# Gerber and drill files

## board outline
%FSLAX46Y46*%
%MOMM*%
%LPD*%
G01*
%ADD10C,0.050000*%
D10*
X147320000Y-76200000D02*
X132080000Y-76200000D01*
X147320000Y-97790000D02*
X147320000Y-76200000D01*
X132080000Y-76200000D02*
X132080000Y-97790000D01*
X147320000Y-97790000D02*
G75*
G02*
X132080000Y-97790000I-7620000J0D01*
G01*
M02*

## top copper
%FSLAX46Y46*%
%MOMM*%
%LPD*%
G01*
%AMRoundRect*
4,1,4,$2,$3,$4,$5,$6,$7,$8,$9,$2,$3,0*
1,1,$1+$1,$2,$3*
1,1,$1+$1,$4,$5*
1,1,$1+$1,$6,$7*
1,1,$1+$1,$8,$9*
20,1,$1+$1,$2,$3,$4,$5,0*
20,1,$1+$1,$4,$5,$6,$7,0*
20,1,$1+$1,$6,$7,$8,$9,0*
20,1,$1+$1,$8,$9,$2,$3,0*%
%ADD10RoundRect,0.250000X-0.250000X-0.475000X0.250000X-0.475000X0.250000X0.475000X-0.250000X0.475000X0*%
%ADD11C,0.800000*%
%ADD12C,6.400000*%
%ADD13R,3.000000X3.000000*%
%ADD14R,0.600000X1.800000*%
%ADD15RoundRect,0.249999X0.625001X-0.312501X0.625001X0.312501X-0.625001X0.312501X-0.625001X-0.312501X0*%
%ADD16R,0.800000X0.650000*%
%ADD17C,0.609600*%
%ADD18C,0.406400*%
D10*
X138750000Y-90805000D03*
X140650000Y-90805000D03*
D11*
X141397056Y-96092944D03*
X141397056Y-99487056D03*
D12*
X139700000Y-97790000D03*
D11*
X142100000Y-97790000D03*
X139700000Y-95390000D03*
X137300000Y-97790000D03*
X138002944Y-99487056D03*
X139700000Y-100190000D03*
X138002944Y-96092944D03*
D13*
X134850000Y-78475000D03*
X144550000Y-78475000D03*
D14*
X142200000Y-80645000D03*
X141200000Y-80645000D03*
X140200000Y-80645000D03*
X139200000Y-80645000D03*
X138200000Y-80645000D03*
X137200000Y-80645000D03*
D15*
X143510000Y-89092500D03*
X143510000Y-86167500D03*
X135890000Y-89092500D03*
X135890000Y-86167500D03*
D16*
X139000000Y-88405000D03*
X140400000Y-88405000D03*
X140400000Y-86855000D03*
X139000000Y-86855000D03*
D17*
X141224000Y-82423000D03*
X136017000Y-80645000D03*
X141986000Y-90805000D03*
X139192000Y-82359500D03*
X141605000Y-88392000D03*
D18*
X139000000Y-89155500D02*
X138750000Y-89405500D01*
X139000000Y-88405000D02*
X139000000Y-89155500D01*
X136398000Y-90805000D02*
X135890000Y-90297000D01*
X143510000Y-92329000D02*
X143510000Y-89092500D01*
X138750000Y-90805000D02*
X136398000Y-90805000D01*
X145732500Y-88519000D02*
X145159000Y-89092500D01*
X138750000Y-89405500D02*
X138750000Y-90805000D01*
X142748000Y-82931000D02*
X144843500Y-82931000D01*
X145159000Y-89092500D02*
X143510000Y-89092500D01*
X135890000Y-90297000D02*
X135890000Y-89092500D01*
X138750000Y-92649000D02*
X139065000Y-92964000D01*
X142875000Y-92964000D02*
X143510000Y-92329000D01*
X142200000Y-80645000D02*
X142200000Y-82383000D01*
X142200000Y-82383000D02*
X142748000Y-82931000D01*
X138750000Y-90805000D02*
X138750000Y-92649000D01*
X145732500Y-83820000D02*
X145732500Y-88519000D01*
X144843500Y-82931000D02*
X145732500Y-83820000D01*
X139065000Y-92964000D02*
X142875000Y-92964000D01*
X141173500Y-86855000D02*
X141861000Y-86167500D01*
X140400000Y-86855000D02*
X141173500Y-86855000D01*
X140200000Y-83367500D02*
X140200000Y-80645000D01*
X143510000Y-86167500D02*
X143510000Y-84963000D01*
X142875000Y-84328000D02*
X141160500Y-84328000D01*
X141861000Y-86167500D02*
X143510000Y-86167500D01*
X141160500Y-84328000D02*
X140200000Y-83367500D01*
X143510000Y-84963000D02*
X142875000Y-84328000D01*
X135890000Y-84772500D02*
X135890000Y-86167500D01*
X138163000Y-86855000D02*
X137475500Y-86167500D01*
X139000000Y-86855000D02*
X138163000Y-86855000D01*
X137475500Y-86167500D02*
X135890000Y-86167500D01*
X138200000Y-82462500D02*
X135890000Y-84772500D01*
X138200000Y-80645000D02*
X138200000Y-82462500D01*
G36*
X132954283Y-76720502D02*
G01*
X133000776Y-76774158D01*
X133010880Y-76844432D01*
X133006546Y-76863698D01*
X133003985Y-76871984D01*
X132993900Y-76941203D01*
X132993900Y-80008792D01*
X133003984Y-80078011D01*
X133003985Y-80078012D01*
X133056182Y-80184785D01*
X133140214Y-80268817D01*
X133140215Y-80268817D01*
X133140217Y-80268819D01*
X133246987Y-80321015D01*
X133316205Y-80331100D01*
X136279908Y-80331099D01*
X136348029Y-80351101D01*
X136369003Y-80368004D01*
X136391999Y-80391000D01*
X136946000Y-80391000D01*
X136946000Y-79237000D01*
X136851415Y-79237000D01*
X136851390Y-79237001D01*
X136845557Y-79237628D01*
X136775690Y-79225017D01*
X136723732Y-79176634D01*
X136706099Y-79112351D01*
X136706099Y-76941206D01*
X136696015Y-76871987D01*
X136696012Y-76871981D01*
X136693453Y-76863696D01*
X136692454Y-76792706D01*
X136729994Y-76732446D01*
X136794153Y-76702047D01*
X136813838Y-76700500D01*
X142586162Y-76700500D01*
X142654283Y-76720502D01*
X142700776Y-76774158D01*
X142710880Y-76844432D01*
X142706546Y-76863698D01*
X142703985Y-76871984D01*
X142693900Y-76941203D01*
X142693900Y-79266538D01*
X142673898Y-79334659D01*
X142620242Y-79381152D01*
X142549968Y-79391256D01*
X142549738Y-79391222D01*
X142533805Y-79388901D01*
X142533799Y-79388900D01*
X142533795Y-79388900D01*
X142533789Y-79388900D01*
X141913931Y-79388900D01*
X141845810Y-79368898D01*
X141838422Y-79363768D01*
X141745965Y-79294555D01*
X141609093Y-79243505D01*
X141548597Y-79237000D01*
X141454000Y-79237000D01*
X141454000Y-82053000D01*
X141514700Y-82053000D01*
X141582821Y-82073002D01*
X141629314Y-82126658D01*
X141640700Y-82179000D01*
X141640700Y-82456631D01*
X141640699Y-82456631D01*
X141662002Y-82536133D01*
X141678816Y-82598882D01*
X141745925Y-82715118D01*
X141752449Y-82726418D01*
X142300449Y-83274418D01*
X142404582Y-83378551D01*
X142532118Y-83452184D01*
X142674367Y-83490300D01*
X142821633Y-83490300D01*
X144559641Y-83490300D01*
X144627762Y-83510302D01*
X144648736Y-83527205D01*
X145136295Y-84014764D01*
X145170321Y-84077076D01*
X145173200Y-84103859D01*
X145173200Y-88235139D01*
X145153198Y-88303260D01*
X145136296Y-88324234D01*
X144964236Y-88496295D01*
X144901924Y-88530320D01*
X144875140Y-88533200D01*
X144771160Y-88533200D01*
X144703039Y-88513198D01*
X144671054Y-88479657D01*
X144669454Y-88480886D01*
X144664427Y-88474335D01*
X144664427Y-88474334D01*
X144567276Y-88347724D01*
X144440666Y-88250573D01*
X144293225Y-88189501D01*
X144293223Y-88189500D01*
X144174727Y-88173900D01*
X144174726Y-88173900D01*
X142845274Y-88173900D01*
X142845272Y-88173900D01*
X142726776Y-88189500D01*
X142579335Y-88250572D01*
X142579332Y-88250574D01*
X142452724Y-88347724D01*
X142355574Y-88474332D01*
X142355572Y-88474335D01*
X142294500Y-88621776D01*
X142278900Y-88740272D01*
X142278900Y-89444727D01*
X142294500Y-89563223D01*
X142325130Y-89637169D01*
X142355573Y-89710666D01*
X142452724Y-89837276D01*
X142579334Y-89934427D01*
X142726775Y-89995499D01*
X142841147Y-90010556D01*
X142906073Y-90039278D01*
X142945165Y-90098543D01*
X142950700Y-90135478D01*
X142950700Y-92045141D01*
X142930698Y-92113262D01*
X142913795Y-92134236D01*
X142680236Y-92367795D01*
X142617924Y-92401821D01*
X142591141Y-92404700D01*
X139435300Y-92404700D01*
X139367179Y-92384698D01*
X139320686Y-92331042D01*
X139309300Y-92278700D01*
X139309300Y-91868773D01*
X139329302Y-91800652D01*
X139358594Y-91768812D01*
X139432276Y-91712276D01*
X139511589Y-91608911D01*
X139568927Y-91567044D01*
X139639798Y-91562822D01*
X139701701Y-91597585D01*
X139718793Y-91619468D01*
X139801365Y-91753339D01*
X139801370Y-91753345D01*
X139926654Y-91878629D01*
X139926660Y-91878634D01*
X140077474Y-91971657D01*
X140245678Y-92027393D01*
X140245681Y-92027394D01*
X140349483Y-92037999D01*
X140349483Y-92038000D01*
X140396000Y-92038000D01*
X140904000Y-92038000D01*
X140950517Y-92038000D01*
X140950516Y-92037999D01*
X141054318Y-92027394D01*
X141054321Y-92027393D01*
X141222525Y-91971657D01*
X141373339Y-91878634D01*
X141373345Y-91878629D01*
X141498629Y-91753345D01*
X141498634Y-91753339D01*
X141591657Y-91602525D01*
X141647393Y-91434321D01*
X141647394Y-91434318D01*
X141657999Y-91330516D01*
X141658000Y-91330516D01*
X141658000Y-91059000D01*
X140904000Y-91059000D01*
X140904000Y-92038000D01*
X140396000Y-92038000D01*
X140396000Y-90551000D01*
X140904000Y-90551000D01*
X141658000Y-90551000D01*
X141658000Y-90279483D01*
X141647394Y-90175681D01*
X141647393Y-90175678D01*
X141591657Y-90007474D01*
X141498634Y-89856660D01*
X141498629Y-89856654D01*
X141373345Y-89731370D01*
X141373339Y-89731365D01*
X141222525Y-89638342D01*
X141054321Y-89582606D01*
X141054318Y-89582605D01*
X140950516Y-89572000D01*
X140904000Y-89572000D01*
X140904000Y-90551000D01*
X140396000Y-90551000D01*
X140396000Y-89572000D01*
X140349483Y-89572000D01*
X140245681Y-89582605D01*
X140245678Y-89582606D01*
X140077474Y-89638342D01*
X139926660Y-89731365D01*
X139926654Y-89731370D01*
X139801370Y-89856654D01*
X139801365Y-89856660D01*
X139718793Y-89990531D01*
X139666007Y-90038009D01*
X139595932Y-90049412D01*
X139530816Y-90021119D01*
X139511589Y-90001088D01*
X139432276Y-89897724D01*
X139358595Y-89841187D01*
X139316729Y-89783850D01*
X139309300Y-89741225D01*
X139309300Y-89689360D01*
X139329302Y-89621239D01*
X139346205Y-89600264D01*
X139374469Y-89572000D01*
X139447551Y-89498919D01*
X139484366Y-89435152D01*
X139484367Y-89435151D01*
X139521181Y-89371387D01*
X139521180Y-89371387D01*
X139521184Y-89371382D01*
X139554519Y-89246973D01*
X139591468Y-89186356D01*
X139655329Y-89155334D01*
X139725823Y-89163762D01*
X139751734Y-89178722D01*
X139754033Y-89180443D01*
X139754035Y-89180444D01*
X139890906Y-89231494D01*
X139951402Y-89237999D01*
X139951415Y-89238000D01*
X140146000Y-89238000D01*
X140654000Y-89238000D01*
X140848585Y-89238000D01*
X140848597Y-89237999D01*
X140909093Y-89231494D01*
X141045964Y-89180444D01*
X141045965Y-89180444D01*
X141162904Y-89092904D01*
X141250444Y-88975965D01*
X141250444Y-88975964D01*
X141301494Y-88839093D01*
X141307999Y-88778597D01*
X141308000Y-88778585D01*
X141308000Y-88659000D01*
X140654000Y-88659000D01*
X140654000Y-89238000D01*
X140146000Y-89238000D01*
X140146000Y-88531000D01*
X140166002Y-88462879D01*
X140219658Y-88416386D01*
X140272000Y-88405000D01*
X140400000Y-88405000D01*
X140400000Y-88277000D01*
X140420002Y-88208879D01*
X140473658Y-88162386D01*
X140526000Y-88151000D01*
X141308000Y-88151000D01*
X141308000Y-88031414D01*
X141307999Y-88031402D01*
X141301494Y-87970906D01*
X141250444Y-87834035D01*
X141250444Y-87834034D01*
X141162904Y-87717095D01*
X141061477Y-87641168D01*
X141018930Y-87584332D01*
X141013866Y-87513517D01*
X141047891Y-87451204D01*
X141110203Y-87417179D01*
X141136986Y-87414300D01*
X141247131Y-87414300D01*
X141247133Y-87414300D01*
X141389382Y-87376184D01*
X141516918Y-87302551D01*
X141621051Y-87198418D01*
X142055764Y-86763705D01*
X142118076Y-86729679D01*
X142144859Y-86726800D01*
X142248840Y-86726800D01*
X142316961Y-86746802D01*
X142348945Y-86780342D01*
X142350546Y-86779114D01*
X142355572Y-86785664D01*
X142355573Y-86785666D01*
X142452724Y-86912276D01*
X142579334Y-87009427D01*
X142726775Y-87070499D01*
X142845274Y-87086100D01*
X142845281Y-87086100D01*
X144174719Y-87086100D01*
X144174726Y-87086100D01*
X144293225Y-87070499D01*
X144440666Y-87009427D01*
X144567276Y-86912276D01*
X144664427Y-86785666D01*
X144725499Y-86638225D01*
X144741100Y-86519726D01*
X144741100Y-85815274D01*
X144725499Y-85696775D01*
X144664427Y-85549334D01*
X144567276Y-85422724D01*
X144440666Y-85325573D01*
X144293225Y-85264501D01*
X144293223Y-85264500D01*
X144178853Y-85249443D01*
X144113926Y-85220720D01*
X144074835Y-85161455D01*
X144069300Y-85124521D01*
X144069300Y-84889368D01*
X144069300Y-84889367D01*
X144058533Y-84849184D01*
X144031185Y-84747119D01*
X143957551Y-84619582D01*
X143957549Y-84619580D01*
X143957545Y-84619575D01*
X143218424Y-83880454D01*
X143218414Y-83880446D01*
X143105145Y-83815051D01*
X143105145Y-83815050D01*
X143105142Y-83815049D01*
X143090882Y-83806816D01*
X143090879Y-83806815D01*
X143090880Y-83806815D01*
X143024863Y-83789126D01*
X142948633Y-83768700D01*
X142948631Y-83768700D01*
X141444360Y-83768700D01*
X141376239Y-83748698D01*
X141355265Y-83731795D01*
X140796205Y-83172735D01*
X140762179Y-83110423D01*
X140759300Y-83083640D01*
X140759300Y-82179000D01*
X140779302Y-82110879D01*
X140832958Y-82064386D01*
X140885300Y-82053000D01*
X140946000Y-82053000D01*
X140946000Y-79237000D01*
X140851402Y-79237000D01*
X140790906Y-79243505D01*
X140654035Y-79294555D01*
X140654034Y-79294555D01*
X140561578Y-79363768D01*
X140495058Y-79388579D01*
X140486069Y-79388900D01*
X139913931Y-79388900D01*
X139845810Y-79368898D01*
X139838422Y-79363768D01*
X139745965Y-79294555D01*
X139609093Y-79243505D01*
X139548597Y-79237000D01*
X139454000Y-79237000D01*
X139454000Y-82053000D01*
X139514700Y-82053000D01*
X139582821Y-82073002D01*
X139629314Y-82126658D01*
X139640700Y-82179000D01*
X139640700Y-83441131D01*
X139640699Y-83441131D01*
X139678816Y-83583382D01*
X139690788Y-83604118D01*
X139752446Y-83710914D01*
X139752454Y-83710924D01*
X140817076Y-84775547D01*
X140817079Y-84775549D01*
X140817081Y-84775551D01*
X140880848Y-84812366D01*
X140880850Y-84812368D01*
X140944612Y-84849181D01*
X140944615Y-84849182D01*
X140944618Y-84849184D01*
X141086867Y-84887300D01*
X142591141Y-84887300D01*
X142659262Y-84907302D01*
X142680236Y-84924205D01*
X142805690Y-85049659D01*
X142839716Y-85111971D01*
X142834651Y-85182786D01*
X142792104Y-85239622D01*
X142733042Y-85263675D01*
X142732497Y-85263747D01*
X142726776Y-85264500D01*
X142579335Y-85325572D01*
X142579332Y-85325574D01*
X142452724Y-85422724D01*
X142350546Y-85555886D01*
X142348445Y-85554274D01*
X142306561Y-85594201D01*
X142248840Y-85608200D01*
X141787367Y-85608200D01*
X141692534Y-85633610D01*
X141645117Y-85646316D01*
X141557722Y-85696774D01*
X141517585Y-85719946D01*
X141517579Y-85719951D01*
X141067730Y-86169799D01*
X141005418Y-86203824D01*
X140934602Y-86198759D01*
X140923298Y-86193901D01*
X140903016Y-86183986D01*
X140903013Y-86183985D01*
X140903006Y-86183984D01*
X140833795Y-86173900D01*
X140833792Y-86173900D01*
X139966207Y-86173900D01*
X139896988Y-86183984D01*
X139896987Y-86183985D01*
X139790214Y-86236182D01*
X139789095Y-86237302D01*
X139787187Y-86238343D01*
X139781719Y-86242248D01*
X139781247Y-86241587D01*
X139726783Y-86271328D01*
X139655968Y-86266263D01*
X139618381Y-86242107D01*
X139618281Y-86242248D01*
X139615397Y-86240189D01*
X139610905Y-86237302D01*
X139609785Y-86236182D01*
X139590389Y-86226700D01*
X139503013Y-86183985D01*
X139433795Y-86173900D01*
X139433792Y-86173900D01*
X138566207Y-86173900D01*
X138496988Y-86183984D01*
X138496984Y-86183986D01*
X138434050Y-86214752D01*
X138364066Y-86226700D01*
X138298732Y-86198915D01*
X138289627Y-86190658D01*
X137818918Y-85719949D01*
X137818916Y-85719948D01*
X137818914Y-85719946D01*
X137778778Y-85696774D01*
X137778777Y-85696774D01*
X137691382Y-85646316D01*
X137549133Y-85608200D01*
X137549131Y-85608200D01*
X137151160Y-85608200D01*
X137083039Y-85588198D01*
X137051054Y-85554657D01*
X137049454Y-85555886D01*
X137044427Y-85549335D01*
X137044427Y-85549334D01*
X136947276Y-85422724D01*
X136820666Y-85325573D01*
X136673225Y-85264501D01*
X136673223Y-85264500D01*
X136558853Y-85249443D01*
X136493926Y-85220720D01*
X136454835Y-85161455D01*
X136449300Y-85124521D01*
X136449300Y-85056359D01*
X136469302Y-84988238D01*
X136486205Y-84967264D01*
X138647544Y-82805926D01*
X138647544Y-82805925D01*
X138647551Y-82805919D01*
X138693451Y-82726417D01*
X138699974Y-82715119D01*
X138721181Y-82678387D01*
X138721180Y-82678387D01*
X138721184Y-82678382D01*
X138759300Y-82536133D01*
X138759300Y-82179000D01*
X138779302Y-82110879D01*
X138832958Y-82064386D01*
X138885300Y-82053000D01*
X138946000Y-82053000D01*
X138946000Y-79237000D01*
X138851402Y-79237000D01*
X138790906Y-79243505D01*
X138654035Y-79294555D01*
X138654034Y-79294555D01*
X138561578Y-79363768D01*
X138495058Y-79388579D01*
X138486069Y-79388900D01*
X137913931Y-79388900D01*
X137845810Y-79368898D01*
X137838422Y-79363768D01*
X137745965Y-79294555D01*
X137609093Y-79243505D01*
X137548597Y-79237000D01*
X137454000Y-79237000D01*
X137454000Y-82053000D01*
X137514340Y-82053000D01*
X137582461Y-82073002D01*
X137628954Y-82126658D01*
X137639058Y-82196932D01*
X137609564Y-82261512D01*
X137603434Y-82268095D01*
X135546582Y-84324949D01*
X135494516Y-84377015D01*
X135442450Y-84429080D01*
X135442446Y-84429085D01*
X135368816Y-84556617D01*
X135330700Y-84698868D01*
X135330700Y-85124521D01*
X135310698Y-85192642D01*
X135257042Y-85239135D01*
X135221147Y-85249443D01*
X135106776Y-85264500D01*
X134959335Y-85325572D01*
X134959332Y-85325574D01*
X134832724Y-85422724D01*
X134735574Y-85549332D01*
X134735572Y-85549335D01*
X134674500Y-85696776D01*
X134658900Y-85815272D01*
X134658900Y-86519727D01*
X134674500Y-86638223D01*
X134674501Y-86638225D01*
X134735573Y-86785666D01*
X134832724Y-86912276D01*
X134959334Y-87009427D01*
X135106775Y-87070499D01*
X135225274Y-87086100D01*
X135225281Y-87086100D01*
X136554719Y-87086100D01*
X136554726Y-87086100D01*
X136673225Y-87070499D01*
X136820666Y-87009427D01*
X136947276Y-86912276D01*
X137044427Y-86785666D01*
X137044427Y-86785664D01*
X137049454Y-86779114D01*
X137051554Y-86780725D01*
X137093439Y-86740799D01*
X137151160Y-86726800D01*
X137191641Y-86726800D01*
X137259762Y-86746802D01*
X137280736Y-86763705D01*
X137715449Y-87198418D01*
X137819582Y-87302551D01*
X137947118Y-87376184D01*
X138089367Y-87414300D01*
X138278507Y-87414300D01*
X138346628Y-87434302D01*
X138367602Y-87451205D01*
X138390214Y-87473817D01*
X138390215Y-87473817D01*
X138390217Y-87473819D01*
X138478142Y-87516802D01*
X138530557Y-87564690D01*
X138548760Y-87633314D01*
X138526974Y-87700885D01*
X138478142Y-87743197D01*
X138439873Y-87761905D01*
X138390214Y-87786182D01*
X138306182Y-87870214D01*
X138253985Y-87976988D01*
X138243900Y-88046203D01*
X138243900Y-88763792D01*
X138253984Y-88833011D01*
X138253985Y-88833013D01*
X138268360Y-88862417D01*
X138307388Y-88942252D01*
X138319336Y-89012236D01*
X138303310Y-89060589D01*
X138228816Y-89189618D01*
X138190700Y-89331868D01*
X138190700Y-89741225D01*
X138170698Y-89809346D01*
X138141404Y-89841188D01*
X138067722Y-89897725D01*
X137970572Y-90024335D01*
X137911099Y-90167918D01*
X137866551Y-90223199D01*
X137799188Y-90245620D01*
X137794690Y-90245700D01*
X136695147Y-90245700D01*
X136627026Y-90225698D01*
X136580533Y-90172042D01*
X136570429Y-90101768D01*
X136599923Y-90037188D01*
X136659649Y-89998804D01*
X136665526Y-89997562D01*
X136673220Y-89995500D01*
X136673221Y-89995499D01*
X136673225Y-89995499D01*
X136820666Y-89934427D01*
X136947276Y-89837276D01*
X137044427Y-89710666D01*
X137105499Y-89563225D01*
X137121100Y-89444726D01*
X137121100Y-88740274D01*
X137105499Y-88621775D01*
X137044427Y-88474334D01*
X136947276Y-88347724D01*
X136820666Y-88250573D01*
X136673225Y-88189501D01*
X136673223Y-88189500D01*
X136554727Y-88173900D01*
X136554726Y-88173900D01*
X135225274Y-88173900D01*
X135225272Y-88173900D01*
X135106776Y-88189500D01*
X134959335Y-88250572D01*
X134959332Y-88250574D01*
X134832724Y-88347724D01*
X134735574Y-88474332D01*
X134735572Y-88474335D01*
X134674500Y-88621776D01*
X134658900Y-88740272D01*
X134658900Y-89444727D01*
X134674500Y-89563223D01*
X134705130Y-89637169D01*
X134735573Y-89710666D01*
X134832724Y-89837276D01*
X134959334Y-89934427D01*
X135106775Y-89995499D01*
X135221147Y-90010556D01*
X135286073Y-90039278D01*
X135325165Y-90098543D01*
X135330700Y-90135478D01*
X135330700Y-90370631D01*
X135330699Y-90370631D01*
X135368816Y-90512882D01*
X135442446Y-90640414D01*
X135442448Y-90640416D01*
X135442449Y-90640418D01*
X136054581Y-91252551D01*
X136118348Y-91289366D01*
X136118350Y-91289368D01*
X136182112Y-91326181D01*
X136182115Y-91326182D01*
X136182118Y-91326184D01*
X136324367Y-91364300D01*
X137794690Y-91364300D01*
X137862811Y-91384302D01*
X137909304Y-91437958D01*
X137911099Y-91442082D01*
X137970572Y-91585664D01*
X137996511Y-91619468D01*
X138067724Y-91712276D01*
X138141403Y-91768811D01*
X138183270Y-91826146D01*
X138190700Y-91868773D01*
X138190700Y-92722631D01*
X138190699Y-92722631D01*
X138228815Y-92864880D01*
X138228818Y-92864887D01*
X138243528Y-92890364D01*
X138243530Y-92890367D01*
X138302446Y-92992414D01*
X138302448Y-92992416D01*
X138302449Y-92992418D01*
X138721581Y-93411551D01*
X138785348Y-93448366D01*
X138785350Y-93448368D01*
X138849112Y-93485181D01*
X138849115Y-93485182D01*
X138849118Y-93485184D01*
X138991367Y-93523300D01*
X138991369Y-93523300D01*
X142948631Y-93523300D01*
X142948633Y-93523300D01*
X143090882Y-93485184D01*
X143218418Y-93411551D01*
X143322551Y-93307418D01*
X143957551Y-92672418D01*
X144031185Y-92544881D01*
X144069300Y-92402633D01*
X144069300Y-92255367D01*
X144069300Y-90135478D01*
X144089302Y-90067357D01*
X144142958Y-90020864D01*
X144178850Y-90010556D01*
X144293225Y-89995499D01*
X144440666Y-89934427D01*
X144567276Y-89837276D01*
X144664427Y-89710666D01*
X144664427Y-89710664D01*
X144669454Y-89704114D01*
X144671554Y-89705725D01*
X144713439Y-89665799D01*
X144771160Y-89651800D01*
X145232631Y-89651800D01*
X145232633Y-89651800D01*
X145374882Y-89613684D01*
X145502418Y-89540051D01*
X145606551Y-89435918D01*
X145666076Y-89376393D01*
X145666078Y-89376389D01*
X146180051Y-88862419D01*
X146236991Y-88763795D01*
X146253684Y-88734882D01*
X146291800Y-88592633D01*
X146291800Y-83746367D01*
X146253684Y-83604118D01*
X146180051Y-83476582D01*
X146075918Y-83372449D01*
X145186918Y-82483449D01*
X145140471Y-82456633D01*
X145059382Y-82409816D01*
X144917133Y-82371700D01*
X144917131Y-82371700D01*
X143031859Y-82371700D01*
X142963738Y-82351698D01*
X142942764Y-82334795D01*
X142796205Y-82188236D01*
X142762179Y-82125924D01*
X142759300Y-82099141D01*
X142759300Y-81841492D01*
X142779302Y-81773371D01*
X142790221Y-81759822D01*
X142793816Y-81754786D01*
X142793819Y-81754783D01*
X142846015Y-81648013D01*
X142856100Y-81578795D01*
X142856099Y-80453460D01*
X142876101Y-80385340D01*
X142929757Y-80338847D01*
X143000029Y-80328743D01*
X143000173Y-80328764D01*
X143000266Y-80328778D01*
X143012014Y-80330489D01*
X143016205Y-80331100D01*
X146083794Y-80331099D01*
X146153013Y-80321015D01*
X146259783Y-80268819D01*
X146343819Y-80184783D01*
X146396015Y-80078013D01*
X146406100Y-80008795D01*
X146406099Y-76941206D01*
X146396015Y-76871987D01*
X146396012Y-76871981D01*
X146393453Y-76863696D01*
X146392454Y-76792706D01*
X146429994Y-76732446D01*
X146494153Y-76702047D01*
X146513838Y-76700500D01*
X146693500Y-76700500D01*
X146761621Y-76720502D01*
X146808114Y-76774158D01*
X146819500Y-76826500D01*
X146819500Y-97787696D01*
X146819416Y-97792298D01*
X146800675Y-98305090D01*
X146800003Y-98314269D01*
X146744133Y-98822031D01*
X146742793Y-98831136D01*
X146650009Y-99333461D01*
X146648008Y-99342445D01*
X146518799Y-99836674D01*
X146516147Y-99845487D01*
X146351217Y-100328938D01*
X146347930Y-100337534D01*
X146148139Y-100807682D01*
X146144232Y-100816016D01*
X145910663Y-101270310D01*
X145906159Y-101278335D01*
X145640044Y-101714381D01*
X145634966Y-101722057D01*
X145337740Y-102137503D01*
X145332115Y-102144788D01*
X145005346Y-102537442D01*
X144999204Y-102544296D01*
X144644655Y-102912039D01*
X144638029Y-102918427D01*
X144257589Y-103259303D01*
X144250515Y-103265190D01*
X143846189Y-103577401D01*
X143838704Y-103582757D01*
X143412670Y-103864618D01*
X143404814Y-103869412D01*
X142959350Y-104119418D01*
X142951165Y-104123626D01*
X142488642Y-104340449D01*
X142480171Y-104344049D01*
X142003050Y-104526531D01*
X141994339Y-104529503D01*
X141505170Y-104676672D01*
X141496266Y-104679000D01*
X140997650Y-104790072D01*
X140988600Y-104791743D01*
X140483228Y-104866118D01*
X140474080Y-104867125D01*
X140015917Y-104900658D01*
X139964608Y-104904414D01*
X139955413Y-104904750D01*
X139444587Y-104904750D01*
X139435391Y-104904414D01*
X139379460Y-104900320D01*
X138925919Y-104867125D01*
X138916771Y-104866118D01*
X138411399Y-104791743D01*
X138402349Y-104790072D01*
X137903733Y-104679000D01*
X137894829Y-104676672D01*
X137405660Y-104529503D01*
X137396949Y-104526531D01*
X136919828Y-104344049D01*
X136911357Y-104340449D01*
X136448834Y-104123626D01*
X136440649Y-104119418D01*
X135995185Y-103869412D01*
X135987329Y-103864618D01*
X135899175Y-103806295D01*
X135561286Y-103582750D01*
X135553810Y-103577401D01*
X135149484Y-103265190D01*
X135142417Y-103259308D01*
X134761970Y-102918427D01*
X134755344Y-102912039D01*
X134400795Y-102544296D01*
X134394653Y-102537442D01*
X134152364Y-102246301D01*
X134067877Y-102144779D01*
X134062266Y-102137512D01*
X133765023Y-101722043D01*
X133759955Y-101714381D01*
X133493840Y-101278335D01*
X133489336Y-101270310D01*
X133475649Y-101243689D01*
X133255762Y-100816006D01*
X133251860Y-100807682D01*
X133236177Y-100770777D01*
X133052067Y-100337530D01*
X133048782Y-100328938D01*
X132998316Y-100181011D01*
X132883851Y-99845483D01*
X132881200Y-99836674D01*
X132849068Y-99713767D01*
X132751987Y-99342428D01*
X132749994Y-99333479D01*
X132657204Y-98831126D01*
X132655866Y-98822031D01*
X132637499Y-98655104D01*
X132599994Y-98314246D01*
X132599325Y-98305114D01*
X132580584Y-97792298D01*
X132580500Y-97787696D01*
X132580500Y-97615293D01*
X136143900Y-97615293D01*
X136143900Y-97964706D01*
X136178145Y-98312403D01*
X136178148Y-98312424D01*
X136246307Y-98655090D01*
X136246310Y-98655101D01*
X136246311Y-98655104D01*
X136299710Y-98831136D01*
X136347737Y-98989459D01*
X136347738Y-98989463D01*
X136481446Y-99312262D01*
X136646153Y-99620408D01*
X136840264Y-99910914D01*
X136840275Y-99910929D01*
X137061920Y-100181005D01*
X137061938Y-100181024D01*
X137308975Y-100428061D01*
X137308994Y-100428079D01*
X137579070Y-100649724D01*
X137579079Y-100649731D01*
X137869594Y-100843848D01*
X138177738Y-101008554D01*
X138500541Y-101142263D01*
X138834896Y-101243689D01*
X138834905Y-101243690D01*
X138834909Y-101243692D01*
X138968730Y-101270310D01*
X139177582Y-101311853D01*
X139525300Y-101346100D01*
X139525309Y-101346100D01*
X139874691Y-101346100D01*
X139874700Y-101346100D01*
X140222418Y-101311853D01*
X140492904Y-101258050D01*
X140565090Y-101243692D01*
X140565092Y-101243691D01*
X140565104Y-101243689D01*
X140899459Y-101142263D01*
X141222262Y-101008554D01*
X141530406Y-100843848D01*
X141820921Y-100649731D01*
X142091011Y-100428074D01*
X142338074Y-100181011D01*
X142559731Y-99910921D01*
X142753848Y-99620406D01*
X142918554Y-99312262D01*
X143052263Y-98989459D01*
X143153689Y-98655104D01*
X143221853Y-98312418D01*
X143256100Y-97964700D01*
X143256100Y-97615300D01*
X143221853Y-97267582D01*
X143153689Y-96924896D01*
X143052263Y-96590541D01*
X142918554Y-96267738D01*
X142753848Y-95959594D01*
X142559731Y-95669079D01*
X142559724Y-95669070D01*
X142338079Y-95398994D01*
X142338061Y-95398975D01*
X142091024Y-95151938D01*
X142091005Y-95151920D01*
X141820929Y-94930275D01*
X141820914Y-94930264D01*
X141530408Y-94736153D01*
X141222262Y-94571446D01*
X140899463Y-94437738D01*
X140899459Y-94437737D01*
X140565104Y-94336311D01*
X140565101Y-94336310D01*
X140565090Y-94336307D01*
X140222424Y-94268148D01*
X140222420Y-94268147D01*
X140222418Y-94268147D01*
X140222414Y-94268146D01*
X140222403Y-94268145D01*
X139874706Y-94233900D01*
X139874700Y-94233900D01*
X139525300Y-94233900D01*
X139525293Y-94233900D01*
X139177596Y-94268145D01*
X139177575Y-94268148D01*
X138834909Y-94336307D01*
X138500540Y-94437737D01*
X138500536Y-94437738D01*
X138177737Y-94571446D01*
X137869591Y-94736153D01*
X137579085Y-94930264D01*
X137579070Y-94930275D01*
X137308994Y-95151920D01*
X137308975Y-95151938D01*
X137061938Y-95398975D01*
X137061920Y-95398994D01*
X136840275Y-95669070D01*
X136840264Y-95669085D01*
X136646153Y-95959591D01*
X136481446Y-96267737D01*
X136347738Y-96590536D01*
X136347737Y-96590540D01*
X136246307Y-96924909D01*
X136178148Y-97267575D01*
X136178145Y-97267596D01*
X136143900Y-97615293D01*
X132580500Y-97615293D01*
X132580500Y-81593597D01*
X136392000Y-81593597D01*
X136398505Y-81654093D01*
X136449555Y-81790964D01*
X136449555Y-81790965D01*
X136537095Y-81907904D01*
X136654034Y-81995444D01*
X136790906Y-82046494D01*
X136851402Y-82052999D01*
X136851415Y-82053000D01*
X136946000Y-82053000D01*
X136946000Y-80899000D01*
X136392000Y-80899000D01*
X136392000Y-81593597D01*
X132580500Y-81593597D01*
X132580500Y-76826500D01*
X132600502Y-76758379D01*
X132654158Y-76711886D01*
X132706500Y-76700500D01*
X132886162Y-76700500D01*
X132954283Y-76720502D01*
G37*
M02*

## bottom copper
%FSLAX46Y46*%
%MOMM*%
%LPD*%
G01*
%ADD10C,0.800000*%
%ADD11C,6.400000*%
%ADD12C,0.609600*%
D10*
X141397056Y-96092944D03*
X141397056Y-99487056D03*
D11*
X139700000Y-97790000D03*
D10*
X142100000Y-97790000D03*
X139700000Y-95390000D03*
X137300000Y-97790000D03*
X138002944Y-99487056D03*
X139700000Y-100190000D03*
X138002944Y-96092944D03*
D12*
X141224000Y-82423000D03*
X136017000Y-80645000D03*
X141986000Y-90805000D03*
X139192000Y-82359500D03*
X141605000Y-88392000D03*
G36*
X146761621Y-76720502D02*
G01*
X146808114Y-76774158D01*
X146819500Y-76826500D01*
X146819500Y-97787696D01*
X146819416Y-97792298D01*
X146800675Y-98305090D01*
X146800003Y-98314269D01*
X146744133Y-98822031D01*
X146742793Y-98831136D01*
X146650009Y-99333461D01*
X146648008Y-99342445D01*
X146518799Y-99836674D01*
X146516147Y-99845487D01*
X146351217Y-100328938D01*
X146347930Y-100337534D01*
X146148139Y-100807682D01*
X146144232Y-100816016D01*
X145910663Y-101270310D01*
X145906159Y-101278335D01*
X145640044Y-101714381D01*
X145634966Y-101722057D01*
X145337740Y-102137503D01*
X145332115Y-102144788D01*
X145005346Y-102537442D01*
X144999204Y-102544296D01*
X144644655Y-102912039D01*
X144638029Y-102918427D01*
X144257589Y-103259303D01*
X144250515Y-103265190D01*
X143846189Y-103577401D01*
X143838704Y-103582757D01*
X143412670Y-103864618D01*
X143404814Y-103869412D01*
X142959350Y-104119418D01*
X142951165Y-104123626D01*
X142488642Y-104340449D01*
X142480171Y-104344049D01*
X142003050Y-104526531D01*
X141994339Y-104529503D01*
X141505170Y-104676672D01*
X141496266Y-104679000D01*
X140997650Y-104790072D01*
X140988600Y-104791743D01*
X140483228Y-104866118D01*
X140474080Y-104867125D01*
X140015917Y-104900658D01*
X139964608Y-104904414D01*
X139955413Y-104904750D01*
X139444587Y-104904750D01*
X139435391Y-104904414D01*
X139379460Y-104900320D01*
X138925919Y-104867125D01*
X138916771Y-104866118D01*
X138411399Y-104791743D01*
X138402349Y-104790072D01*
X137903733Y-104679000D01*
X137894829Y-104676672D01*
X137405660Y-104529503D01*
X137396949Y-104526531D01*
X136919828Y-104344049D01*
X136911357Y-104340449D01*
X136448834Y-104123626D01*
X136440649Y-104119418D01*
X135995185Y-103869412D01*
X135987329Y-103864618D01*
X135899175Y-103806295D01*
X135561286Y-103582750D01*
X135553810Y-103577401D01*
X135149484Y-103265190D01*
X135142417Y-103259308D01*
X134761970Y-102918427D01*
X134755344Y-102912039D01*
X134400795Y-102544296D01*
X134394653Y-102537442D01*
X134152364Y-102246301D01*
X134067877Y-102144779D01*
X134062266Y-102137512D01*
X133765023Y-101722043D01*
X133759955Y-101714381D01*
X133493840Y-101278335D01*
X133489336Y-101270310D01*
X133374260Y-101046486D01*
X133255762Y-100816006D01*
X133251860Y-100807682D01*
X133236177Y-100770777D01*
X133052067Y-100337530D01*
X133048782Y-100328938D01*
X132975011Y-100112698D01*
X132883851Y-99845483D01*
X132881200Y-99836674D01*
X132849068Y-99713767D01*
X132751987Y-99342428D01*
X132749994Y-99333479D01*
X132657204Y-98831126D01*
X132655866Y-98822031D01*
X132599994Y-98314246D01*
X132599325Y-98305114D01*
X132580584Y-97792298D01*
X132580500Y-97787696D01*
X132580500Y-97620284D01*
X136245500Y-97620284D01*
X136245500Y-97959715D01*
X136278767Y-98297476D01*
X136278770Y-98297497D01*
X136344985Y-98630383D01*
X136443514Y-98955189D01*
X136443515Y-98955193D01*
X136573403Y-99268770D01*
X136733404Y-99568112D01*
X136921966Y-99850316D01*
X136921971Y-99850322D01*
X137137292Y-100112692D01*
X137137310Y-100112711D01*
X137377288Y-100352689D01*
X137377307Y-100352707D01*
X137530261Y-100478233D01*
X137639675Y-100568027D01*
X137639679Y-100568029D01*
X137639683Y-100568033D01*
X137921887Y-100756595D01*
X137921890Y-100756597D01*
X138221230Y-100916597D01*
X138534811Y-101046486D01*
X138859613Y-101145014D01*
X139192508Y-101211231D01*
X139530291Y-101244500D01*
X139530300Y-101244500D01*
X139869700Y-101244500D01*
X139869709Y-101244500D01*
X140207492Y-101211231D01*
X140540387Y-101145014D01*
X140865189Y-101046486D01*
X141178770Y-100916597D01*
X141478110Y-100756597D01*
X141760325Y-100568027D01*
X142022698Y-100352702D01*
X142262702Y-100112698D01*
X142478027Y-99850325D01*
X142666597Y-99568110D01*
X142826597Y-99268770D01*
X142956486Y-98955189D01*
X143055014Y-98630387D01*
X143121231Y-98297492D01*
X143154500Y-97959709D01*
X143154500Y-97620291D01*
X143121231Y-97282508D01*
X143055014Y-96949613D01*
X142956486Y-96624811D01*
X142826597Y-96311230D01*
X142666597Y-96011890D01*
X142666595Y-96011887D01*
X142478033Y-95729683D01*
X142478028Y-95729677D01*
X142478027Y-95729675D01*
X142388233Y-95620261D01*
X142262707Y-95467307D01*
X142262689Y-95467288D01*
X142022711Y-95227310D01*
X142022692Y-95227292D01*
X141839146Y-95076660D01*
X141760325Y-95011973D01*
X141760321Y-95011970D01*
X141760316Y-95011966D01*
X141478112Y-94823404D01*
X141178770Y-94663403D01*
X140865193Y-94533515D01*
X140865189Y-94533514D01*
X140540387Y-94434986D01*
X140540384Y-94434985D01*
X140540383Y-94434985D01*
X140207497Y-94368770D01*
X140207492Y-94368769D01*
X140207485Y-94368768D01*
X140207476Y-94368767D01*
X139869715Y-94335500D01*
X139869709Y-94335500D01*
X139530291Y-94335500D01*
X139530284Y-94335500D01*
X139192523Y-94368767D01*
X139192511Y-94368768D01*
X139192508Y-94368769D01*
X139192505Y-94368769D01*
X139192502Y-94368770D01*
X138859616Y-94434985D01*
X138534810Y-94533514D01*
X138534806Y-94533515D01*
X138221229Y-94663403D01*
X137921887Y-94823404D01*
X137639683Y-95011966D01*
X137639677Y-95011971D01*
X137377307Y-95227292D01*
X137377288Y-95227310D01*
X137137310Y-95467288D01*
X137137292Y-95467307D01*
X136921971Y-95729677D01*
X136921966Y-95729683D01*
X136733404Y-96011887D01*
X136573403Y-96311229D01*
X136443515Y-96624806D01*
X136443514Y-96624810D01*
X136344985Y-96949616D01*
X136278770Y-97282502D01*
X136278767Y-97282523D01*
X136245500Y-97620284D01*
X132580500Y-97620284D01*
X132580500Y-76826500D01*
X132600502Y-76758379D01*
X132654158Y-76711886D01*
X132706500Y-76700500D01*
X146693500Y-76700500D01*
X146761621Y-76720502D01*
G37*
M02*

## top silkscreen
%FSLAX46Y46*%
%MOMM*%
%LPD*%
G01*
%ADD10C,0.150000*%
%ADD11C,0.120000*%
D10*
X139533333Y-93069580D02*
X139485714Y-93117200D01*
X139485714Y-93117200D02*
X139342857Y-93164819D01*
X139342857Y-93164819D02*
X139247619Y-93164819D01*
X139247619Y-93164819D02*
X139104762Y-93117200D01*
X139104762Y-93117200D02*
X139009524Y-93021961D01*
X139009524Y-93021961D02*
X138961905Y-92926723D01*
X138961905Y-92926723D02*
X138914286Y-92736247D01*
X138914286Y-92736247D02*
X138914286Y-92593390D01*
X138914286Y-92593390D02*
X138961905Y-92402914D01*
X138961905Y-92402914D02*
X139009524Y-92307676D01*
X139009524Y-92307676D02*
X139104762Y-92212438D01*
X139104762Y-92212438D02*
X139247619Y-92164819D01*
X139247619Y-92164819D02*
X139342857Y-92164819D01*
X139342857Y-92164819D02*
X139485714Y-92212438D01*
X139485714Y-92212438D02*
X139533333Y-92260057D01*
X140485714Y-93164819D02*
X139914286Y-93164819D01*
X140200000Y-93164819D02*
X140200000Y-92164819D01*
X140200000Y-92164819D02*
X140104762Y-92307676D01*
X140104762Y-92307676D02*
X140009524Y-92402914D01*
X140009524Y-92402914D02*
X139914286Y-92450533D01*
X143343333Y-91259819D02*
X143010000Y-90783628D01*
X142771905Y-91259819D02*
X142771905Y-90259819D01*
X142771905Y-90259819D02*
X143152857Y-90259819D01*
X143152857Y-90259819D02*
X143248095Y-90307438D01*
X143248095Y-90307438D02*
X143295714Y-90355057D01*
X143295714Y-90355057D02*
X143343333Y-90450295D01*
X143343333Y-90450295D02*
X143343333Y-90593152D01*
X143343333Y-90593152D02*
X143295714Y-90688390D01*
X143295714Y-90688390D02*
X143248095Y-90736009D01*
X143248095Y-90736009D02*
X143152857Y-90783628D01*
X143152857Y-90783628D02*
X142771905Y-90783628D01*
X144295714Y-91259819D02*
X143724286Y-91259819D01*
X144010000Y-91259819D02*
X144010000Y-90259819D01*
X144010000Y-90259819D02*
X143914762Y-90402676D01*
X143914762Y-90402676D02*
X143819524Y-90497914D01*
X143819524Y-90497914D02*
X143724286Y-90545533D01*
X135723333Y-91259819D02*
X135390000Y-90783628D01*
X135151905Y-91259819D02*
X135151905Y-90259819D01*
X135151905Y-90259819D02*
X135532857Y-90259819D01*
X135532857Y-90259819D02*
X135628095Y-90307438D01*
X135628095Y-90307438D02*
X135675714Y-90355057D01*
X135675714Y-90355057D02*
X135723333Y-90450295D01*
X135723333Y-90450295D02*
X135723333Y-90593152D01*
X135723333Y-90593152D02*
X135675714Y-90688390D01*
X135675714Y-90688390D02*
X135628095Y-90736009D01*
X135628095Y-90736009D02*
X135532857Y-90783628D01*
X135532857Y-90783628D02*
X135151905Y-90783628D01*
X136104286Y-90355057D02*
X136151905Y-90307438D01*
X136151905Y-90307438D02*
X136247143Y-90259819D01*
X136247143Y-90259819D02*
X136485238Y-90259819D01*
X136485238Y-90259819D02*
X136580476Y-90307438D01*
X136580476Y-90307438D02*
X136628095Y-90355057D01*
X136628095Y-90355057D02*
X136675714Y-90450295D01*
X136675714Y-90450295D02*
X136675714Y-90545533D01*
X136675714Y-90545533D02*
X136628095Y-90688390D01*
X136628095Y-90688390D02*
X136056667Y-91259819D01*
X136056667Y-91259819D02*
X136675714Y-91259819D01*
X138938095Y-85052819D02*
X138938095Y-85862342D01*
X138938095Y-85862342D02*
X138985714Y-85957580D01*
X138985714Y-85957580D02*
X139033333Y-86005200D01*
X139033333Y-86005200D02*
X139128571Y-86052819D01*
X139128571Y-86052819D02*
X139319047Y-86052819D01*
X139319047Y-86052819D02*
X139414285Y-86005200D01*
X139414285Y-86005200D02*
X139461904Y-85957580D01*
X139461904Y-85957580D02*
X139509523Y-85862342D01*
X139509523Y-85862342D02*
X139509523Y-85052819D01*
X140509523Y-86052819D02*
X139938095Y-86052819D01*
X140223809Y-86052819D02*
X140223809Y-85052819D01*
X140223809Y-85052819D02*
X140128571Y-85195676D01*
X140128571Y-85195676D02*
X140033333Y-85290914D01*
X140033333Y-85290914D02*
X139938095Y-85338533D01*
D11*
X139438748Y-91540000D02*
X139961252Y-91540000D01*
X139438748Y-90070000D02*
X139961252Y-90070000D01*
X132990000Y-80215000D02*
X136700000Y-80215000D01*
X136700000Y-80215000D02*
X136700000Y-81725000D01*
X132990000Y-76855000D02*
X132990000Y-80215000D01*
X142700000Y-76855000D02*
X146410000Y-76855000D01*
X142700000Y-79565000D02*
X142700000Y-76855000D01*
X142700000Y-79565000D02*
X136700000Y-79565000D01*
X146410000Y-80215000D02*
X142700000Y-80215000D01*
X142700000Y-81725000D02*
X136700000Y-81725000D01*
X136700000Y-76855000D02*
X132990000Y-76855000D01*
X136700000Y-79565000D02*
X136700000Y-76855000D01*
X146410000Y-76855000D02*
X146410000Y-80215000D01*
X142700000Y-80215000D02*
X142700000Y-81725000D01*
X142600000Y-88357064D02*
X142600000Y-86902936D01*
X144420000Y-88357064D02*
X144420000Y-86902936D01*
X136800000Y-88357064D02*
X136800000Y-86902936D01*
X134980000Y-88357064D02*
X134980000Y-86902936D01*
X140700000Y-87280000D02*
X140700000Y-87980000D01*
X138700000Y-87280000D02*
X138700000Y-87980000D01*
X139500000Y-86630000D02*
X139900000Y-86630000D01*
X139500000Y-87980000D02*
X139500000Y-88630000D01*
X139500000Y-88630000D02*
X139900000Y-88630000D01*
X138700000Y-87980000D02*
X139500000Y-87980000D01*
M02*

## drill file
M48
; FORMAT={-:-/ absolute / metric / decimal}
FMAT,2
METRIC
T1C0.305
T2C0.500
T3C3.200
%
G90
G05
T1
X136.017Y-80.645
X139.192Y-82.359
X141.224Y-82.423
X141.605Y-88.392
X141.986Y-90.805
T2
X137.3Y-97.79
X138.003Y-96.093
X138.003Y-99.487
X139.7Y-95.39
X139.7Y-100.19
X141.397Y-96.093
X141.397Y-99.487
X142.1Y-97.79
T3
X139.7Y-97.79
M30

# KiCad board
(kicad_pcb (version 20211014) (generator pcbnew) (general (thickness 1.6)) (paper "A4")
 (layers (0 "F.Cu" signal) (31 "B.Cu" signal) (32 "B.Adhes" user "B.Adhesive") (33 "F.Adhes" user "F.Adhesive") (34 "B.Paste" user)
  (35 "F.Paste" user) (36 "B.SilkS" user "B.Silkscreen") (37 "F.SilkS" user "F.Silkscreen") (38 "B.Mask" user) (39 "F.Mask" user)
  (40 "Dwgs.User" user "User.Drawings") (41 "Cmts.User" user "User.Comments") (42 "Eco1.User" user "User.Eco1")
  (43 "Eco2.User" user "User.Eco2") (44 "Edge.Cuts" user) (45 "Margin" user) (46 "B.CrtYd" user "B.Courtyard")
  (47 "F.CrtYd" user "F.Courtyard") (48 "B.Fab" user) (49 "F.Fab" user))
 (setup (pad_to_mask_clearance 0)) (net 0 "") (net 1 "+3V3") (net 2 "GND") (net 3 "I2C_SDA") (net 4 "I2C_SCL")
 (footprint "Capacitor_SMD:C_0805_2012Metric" (layer "F.Cu") (at 139.7 90.805)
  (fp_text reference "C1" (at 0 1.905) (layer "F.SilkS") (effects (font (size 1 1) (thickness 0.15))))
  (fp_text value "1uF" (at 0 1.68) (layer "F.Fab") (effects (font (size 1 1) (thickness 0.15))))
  (fp_line (start -0.261252 0.735) (end 0.261252 0.735) (layer "F.SilkS") (width 0.12))
  (fp_line (start -0.261252 -0.735) (end 0.261252 -0.735) (layer "F.SilkS") (width 0.12))
  (pad "1" smd roundrect locked (at -0.95 0) (size 1 1.45) (layers "F.Cu" "F.Paste" "F.Mask") (roundrect_rratio 0.25) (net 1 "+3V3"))
  (pad "2" smd roundrect locked (at 0.95 0) (size 1 1.45) (layers "F.Cu" "F.Paste" "F.Mask") (roundrect_rratio 0.25) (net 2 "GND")))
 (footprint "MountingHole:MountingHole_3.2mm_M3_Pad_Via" (layer "F.Cu") (at 139.7 97.79)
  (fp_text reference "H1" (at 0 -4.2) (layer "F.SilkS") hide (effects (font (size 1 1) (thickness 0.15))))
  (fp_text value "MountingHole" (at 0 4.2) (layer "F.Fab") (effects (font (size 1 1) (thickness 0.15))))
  (pad "1" thru_hole circle locked (at 1.697056 -1.697056) (size 0.8 0.8) (drill 0.5) (layers *.Cu *.Mask))
  (pad "1" thru_hole circle locked (at 1.697056 1.697056) (size 0.8 0.8) (drill 0.5) (layers *.Cu *.Mask))
  (pad "1" thru_hole circle locked (at 0 0) (size 6.4 6.4) (drill 3.2) (layers *.Cu *.Mask))
  (pad "1" thru_hole circle locked (at 2.4 0) (size 0.8 0.8) (drill 0.5) (layers *.Cu *.Mask))
  (pad "1" thru_hole circle locked (at 0 -2.4) (size 0.8 0.8) (drill 0.5) (layers *.Cu *.Mask))
  (pad "1" thru_hole circle locked (at -2.4 0) (size 0.8 0.8) (drill 0.5) (layers *.Cu *.Mask))
  (pad "1" thru_hole circle locked (at -1.697056 1.697056) (size 0.8 0.8) (drill 0.5) (layers *.Cu *.Mask))
  (pad "1" thru_hole circle locked (at 0 2.4) (size 0.8 0.8) (drill 0.5) (layers *.Cu *.Mask))
  (pad "1" thru_hole circle locked (at -1.697056 -1.697056) (size 0.8 0.8) (drill 0.5) (layers *.Cu *.Mask)))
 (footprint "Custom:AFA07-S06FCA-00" (layer "F.Cu") (at 139.7 80.645 180)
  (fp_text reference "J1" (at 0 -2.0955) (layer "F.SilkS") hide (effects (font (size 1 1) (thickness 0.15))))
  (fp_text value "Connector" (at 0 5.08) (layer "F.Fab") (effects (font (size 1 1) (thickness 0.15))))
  (fp_line (start 6.71 0.43) (end 3 0.43) (layer "F.SilkS") (width 0.12))
  (fp_line (start 3 0.43) (end 3 -1.08) (layer "F.SilkS") (width 0.12))
  (fp_line (start 6.71 3.79) (end 6.71 0.43) (layer "F.SilkS") (width 0.12))
  (fp_line (start -3 3.79) (end -6.71 3.79) (layer "F.SilkS") (width 0.12))
  (fp_line (start -3 1.08) (end -3 3.79) (layer "F.SilkS") (width 0.12))
  (fp_line (start -3 1.08) (end 3 1.08) (layer "F.SilkS") (width 0.12))
  (fp_line (start -6.71 0.43) (end -3 0.43) (layer "F.SilkS") (width 0.12))
  (fp_line (start -3 -1.08) (end 3 -1.08) (layer "F.SilkS") (width 0.12))
  (fp_line (start 3 3.79) (end 6.71 3.79) (layer "F.SilkS") (width 0.12))
  (fp_line (start 3 1.08) (end 3 3.79) (layer "F.SilkS") (width 0.12))
  (fp_line (start -6.71 3.79) (end -6.71 0.43) (layer "F.SilkS") (width 0.12))
  (fp_line (start -3 0.43) (end -3 -1.08) (layer "F.SilkS") (width 0.12))
  (pad "" smd rect locked (at 4.85 2.17 180) (size 3 3) (layers "F.Cu" "F.Paste" "F.Mask"))
  (pad "" smd rect locked (at -4.85 2.17 180) (size 3 3) (layers "F.Cu" "F.Paste" "F.Mask"))
  (pad "1" smd rect locked (at -2.5 0 180) (size 0.6 1.8) (layers "F.Cu" "F.Paste" "F.Mask") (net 1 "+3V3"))
  (pad "2" smd rect locked (at -1.5 0 180) (size 0.6 1.8) (layers "F.Cu" "F.Paste" "F.Mask") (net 2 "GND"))
  (pad "3" smd rect locked (at -0.5 0 180) (size 0.6 1.8) (layers "F.Cu" "F.Paste" "F.Mask") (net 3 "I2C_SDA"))
  (pad "4" smd rect locked (at 0.5 0 180) (size 0.6 1.8) (layers "F.Cu" "F.Paste" "F.Mask") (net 2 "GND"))
  (pad "5" smd rect locked (at 1.5 0 180) (size 0.6 1.8) (layers "F.Cu" "F.Paste" "F.Mask") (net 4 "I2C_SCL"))
  (pad "6" smd rect locked (at 2.5 0 180) (size 0.6 1.8) (layers "F.Cu" "F.Paste" "F.Mask") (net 2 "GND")))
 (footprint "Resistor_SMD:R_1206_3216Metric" (layer "F.Cu") (at 143.51 87.63 90)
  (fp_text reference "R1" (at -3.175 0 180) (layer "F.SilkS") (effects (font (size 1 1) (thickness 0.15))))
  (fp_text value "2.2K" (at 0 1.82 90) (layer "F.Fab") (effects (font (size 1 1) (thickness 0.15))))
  (fp_line (start -0.727064 -0.91) (end 0.727064 -0.91) (layer "F.SilkS") (width 0.12))
  (fp_line (start -0.727064 0.91) (end 0.727064 0.91) (layer "F.SilkS") (width 0.12))
  (pad "1" smd roundrect locked (at -1.4625 0 90) (size 1.125 1.75) (layers "F.Cu" "F.Paste" "F.Mask") (roundrect_rratio 0.2222213333)
   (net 1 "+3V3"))
  (pad "2" smd roundrect locked (at 1.4625 0 90) (size 1.125 1.75) (layers "F.Cu" "F.Paste" "F.Mask") (roundrect_rratio 0.2222213333)
   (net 3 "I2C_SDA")))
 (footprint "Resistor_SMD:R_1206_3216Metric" (layer "F.Cu") (at 135.89 87.63 90)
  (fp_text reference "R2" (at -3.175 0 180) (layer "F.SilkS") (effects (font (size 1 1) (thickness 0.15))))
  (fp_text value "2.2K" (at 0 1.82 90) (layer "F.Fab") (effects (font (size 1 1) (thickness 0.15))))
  (fp_line (start -0.727064 0.91) (end 0.727064 0.91) (layer "F.SilkS") (width 0.12))
  (fp_line (start -0.727064 -0.91) (end 0.727064 -0.91) (layer "F.SilkS") (width 0.12))
  (pad "1" smd roundrect locked (at -1.4625 0 90) (size 1.125 1.75) (layers "F.Cu" "F.Paste" "F.Mask") (roundrect_rratio 0.2222213333)
   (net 1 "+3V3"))
  (pad "2" smd roundrect locked (at 1.4625 0 90) (size 1.125 1.75) (layers "F.Cu" "F.Paste" "F.Mask") (roundrect_rratio 0.2222213333)
   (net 4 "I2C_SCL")))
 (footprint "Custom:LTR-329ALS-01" (layer "F.Cu") (at 139.7 87.63)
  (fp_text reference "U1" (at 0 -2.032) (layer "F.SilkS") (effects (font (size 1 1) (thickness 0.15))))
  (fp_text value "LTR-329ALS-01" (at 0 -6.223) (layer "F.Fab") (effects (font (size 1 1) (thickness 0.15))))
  (fp_line (start 1 -0.35) (end 1 0.35) (layer "F.SilkS") (width 0.12))
  (fp_line (start -1 -0.35) (end -1 0.35) (layer "F.SilkS") (width 0.12))
  (fp_line (start -0.2 -1) (end 0.2 -1) (layer "F.SilkS") (width 0.12))
  (fp_line (start -0.2 0.35) (end -0.2 1) (layer "F.SilkS") (width 0.12))
  (fp_line (start -0.2 1) (end 0.2 1) (layer "F.SilkS") (width 0.12))
  (fp_line (start -1 0.35) (end -0.2 0.35) (layer "F.SilkS") (width 0.12))
  (pad "1" smd rect locked (at -0.7 0.775) (size 0.8 0.65) (layers "F.Cu" "F.Paste" "F.Mask") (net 1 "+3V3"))
  (pad "2" smd rect locked (at 0.7 0.775) (size 0.8 0.65) (layers "F.Cu" "F.Paste" "F.Mask") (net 2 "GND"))
  (pad "3" smd rect locked (at 0.7 -0.775) (size 0.8 0.65) (layers "F.Cu" "F.Paste" "F.Mask") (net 3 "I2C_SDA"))
  (pad "4" smd rect locked (at -0.7 -0.775) (size 0.8 0.65) (layers "F.Cu" "F.Paste" "F.Mask") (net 4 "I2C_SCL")))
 (gr_line (start 147.32 76.2) (end 132.08 76.2) (layer "Edge.Cuts") (width 0.05))
 (gr_line (start 147.32 97.79) (end 147.32 76.2) (layer "Edge.Cuts") (width 0.05))
 (gr_line (start 132.08 76.2) (end 132.08 97.79) (layer "Edge.Cuts") (width 0.05))
 (gr_arc (start 147.32 97.79) (mid 139.7 105.41) (end 132.08 97.79) (layer "Edge.Cuts") (width 0.05))
 (via (at 141.224 82.423) (size 0.6096) (drill 0.3048) (layers "F.Cu" "B.Cu") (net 2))
 (via (at 136.017 80.645) (size 0.6096) (drill 0.3048) (layers "F.Cu" "B.Cu") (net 2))
 (via (at 141.986 90.805) (size 0.6096) (drill 0.3048) (layers "F.Cu" "B.Cu") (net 2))
 (via (at 139.192 82.3595) (size 0.6096) (drill 0.3048) (layers "F.Cu" "B.Cu") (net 2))
 (via (at 141.605 88.392) (size 0.6096) (drill 0.3048) (layers "F.Cu" "B.Cu") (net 2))
 (segment (start 139 89.1555) (end 138.75 89.4055) (width 0.4064) (layer "F.Cu") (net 1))
 (segment (start 139 88.405) (end 139 89.1555) (width 0.4064) (layer "F.Cu") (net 1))
 (segment (start 136.398 90.805) (end 135.89 90.297) (width 0.4064) (layer "F.Cu") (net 1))
 (segment (start 143.51 92.329) (end 143.51 89.0925) (width 0.4064) (layer "F.Cu") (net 1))
 (segment (start 138.75 90.805) (end 136.398 90.805) (width 0.4064) (layer "F.Cu") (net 1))
 (segment (start 145.7325 88.519) (end 145.159 89.0925) (width 0.4064) (layer "F.Cu") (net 1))
 (segment (start 138.75 89.4055) (end 138.75 90.805) (width 0.4064) (layer "F.Cu") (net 1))
 (segment (start 142.748 82.931) (end 144.8435 82.931) (width 0.4064) (layer "F.Cu") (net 1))
 (segment (start 145.159 89.0925) (end 143.51 89.0925) (width 0.4064) (layer "F.Cu") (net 1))
 (segment (start 135.89 90.297) (end 135.89 89.0925) (width 0.4064) (layer "F.Cu") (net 1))
 (segment (start 138.75 92.649) (end 139.065 92.964) (width 0.4064) (layer "F.Cu") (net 1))
 (segment (start 142.875 92.964) (end 143.51 92.329) (width 0.4064) (layer "F.Cu") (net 1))
 (segment (start 142.2 80.645) (end 142.2 82.383) (width 0.4064) (layer "F.Cu") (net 1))
 (segment (start 142.2 82.383) (end 142.748 82.931) (width 0.4064) (layer "F.Cu") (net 1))
 (segment (start 138.75 90.805) (end 138.75 92.649) (width 0.4064) (layer "F.Cu") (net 1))
 (segment (start 145.7325 83.82) (end 145.7325 88.519) (width 0.4064) (layer "F.Cu") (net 1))
 (segment (start 144.8435 82.931) (end 145.7325 83.82) (width 0.4064) (layer "F.Cu") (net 1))
 (segment (start 139.065 92.964) (end 142.875 92.964) (width 0.4064) (layer "F.Cu") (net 1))
 (segment (start 141.1735 86.855) (end 141.861 86.1675) (width 0.4064) (layer "F.Cu") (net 3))
 (segment (start 140.4 86.855) (end 141.1735 86.855) (width 0.4064) (layer "F.Cu") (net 3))
 (segment (start 140.2 83.3675) (end 140.2 80.645) (width 0.4064) (layer "F.Cu") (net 3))
 (segment (start 143.51 86.1675) (end 143.51 84.963) (width 0.4064) (layer "F.Cu") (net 3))
 (segment (start 142.875 84.328) (end 141.1605 84.328) (width 0.4064) (layer "F.Cu") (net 3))
 (segment (start 141.861 86.1675) (end 143.51 86.1675) (width 0.4064) (layer "F.Cu") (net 3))
 (segment (start 141.1605 84.328) (end 140.2 83.3675) (width 0.4064) (layer "F.Cu") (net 3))
 (segment (start 143.51 84.963) (end 142.875 84.328) (width 0.4064) (layer "F.Cu") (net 3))
 (segment (start 135.89 84.7725) (end 135.89 86.1675) (width 0.4064) (layer "F.Cu") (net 4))
 (segment (start 138.163 86.855) (end 137.4755 86.1675) (width 0.4064) (layer "F.Cu") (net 4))
 (segment (start 139 86.855) (end 138.163 86.855) (width 0.4064) (layer "F.Cu") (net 4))
 (segment (start 137.4755 86.1675) (end 135.89 86.1675) (width 0.4064) (layer "F.Cu") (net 4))
 (segment (start 138.2 82.4625) (end 135.89 84.7725) (width 0.4064) (layer "F.Cu") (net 4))
 (segment (start 138.2 80.645) (end 138.2 82.4625) (width 0.4064) (layer "F.Cu") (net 4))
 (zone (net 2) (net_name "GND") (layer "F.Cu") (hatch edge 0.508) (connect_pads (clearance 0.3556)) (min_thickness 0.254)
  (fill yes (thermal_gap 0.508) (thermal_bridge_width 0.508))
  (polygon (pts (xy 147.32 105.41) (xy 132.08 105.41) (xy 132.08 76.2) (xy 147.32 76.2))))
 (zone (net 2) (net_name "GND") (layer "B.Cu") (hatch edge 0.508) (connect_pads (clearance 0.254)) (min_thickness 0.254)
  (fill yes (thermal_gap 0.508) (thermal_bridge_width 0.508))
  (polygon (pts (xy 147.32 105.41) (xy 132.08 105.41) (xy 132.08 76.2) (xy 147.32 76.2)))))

